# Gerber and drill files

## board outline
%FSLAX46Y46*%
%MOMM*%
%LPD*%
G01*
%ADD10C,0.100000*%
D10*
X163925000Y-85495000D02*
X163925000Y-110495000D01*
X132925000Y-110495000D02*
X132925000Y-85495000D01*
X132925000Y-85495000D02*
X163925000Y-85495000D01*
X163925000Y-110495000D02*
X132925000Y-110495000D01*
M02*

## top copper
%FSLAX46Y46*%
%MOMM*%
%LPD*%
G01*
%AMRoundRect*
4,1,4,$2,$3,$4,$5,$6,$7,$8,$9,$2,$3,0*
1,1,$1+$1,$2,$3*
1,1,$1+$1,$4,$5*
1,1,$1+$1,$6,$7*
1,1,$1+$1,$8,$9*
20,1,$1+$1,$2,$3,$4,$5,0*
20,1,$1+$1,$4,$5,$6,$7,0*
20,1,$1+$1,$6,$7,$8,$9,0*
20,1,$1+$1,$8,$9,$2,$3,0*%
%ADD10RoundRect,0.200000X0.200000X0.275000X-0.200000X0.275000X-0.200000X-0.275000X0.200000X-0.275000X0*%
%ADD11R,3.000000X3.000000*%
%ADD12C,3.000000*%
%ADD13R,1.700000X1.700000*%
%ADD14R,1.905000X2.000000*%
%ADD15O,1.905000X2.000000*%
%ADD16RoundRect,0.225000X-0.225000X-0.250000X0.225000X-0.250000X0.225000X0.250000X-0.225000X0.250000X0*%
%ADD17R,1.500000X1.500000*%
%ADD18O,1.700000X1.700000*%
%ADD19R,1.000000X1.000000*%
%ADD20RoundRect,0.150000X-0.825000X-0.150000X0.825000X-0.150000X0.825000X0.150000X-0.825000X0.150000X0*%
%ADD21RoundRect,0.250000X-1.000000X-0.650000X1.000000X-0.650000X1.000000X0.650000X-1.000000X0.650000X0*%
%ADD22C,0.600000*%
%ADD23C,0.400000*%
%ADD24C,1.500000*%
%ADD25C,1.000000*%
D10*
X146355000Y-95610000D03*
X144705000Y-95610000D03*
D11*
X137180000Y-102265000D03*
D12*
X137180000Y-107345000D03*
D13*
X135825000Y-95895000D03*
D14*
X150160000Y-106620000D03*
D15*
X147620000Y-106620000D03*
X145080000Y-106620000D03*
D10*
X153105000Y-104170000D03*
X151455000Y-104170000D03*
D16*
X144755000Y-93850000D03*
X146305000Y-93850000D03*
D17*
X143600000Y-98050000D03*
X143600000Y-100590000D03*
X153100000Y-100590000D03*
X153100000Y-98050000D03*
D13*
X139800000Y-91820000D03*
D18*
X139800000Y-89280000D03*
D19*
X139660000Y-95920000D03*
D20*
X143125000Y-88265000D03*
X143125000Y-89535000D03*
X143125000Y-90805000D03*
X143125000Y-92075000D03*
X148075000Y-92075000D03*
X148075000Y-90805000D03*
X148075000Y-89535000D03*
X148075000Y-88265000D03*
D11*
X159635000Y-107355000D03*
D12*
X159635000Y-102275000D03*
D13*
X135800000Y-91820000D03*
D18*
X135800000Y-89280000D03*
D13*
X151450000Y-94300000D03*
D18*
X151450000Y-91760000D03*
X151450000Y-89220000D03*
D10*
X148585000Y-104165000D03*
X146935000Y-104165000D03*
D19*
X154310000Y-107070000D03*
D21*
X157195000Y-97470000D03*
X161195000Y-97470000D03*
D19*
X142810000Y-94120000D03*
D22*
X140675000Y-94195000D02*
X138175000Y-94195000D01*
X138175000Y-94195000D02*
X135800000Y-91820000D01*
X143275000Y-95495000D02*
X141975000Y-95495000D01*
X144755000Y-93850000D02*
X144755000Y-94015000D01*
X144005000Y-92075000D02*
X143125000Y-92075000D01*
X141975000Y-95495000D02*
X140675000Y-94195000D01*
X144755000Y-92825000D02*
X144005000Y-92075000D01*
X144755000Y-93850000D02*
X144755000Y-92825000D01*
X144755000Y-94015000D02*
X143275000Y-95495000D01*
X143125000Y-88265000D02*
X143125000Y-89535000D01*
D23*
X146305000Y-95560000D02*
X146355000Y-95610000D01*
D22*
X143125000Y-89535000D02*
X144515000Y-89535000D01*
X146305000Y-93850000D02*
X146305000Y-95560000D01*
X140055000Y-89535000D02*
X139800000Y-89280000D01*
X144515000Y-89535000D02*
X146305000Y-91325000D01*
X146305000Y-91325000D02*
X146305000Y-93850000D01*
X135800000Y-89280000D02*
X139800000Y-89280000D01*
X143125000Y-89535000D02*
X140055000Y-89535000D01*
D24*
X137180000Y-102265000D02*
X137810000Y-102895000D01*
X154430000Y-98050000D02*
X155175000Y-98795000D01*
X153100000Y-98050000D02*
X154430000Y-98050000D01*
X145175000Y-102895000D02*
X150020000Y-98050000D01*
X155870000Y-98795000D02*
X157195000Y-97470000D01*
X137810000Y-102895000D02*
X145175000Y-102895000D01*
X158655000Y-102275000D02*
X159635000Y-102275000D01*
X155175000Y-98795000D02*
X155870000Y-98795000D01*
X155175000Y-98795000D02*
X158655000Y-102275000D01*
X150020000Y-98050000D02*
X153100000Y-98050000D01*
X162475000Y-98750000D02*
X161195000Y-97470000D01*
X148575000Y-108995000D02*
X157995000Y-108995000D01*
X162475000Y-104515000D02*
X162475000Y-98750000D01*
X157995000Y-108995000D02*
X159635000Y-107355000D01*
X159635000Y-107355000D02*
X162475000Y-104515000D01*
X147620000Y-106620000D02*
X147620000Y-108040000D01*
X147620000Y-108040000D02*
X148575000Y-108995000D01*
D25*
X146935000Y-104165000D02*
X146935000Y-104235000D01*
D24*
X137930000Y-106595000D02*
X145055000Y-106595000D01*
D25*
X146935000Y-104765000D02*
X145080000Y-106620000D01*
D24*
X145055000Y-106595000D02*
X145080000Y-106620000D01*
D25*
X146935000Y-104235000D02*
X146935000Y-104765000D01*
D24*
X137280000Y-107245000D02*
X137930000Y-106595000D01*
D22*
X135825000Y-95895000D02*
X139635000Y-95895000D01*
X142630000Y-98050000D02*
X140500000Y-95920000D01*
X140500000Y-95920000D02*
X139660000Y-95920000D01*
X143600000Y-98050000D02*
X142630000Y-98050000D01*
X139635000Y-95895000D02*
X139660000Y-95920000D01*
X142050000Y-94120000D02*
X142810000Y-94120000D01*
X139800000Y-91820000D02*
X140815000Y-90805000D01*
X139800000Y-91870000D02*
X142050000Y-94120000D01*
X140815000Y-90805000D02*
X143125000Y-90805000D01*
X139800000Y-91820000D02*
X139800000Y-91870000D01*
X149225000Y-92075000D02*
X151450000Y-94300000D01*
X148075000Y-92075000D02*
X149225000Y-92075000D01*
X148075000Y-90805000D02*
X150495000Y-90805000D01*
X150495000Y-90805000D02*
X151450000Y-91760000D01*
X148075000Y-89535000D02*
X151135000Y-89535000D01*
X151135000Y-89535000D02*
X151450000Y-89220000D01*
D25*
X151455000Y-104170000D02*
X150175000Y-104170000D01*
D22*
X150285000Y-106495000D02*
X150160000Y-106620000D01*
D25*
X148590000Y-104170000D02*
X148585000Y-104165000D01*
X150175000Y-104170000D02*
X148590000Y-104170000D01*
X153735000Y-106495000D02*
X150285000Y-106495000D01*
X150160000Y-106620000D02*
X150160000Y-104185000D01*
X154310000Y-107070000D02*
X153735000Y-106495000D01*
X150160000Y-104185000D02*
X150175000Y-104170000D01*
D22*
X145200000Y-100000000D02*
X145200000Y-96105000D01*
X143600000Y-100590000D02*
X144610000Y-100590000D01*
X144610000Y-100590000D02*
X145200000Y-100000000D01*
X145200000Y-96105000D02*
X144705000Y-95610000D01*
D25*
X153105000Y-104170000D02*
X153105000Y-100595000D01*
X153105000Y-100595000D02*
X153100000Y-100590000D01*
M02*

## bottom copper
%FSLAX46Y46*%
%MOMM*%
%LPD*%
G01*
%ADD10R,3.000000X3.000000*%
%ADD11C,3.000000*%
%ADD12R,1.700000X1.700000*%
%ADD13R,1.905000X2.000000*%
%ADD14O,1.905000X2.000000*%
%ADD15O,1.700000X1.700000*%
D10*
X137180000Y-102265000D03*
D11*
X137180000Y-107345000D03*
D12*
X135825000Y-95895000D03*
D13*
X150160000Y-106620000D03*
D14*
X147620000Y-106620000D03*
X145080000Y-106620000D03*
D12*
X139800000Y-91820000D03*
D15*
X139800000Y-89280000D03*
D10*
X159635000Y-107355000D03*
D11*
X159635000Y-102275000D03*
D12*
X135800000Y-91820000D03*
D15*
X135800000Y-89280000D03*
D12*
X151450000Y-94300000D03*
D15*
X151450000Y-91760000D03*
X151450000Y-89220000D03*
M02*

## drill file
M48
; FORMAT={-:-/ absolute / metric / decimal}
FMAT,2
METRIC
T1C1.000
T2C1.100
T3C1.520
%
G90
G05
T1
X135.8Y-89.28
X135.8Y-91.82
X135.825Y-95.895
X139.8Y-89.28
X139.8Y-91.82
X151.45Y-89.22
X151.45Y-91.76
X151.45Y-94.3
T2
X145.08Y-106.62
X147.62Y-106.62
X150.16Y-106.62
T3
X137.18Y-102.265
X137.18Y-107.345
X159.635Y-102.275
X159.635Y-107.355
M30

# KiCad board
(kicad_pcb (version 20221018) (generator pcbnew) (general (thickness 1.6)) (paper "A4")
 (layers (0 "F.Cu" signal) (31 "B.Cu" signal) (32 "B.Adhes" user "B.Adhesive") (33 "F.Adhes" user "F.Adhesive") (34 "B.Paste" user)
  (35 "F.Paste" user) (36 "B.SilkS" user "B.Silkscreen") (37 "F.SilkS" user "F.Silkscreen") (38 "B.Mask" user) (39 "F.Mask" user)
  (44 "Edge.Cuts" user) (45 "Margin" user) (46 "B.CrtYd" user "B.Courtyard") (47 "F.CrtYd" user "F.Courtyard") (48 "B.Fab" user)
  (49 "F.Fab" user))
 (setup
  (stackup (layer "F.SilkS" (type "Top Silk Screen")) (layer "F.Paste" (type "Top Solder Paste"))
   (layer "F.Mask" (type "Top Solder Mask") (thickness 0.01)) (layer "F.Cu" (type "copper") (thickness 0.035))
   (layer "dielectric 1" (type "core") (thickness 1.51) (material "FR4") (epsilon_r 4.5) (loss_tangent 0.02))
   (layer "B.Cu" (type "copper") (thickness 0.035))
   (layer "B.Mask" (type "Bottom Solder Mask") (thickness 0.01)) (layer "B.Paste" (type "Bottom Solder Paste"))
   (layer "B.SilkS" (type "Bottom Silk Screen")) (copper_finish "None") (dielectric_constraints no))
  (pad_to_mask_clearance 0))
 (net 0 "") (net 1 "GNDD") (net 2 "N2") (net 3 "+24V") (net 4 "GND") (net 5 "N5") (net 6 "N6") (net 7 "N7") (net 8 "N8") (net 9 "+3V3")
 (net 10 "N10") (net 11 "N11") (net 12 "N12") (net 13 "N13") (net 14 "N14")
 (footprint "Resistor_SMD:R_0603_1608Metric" (layer "F.Cu") (at 145.53 95.61 180)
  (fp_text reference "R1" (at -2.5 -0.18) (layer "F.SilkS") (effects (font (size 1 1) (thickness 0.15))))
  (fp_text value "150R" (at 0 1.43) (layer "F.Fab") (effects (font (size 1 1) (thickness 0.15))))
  (pad "1" smd roundrect (at -0.825 0 180) (size 0.8 0.95) (layers "F.Cu" "F.Paste" "F.Mask") (roundrect_rratio 0.25) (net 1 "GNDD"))
  (pad "2" smd roundrect (at 0.825 0 180) (size 0.8 0.95) (layers "F.Cu" "F.Paste" "F.Mask") (roundrect_rratio 0.25) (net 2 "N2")))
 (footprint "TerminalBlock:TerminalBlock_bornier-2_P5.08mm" (layer "F.Cu") (at 137.18 102.265 -90)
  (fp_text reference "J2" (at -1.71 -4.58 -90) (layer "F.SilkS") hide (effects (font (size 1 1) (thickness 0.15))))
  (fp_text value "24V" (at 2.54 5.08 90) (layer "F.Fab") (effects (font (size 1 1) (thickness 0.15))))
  (pad "1" thru_hole rect (at 0 0 270) (size 3 3) (drill 1.52) (layers "*.Cu" "*.Mask") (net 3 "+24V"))
  (pad "2" thru_hole circle (at 5.08 0 270) (size 3 3) (drill 1.52) (layers "*.Cu" "*.Mask") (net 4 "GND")))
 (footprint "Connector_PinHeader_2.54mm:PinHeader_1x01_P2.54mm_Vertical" (layer "F.Cu") (at 135.825 95.895)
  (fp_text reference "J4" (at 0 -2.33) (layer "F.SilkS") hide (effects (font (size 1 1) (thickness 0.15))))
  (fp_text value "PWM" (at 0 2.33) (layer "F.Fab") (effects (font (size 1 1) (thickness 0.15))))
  (pad "1" thru_hole rect (at 0 0) (size 1.7 1.7) (drill 1) (layers "*.Cu" "*.Mask") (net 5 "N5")))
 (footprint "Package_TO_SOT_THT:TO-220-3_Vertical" (layer "F.Cu") (at 150.16 106.62 180)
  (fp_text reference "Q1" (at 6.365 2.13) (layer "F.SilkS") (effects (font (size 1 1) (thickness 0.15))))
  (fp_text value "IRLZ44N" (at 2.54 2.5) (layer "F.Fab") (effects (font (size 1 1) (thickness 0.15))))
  (pad "1" thru_hole rect (at 0 0 180) (size 1.905 2) (drill 1.1) (layers "*.Cu" "*.Mask") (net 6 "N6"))
  (pad "2" thru_hole oval (at 2.54 0 180) (size 1.905 2) (drill 1.1) (layers "*.Cu" "*.Mask") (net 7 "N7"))
  (pad "3" thru_hole oval (at 5.08 0 180) (size 1.905 2) (drill 1.1) (layers "*.Cu" "*.Mask") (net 4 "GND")))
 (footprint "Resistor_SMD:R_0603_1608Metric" (layer "F.Cu") (at 152.28 104.17 180)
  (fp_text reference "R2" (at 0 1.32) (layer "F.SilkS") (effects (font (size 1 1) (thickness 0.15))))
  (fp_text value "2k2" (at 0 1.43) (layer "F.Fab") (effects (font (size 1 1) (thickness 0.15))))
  (pad "1" smd roundrect (at -0.825 0 180) (size 0.8 0.95) (layers "F.Cu" "F.Paste" "F.Mask") (roundrect_rratio 0.25) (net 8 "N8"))
  (pad "2" smd roundrect (at 0.825 0 180) (size 0.8 0.95) (layers "F.Cu" "F.Paste" "F.Mask") (roundrect_rratio 0.25) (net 6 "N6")))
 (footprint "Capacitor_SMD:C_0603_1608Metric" (layer "F.Cu") (at 145.53 93.85)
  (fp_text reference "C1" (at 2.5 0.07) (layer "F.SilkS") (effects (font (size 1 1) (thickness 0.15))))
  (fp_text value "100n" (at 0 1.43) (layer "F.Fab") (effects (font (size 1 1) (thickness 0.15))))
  (pad "1" smd roundrect (at -0.775 0) (size 0.9 0.95) (layers "F.Cu" "F.Paste" "F.Mask") (roundrect_rratio 0.25) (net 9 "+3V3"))
  (pad "2" smd roundrect (at 0.775 0) (size 0.9 0.95) (layers "F.Cu" "F.Paste" "F.Mask") (roundrect_rratio 0.25) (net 1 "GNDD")))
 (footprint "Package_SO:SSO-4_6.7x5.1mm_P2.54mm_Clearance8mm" (layer "F.Cu") (at 148.35 99.32)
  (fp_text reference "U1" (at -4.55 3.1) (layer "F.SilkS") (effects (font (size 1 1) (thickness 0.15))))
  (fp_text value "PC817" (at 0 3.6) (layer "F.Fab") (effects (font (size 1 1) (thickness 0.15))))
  (pad "1" smd rect (at -4.75 -1.27) (size 1.5 1.5) (layers "F.Cu" "F.Paste" "F.Mask") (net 5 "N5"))
  (pad "2" smd rect (at -4.75 1.27) (size 1.5 1.5) (layers "F.Cu" "F.Paste" "F.Mask") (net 2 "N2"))
  (pad "3" smd rect (at 4.75 1.27) (size 1.5 1.5) (layers "F.Cu" "F.Paste" "F.Mask") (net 8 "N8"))
  (pad "4" smd rect (at 4.75 -1.27) (size 1.5 1.5) (layers "F.Cu" "F.Paste" "F.Mask") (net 3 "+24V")))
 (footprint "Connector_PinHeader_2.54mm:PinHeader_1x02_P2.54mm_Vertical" (layer "F.Cu") (at 139.8 91.82 180)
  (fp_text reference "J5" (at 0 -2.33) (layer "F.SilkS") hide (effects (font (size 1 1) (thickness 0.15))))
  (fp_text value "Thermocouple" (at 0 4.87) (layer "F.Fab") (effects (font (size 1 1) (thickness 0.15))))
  (pad "1" thru_hole rect (at 0 0 180) (size 1.7 1.7) (drill 1) (layers "*.Cu" "*.Mask") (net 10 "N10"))
  (pad "2" thru_hole oval (at 0 2.54 180) (size 1.7 1.7) (drill 1) (layers "*.Cu" "*.Mask") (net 1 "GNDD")))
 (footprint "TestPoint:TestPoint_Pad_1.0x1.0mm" (layer "F.Cu") (at 139.66 95.92)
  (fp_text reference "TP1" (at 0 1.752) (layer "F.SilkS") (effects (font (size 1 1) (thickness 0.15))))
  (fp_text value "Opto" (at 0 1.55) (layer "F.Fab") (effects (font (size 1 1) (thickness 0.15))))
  (pad "1" smd rect (at 0 0) (size 1 1) (layers "F.Cu" "F.Mask") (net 5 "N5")))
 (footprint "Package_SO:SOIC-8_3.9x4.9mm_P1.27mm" (layer "F.Cu") (at 145.6 90.17)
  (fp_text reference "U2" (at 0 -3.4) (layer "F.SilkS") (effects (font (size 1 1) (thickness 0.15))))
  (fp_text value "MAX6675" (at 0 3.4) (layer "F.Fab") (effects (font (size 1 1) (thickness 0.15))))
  (pad "1" smd roundrect (at -2.475 -1.905) (size 1.95 0.6) (layers "F.Cu" "F.Paste" "F.Mask") (roundrect_rratio 0.25) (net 1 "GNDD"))
  (pad "2" smd roundrect (at -2.475 -0.635) (size 1.95 0.6) (layers "F.Cu" "F.Paste" "F.Mask") (roundrect_rratio 0.25) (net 1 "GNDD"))
  (pad "3" smd roundrect (at -2.475 0.635) (size 1.95 0.6) (layers "F.Cu" "F.Paste" "F.Mask") (roundrect_rratio 0.25) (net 10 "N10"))
  (pad "4" smd roundrect (at -2.475 1.905) (size 1.95 0.6) (layers "F.Cu" "F.Paste" "F.Mask") (roundrect_rratio 0.25) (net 9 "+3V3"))
  (pad "5" smd roundrect (at 2.475 1.905) (size 1.95 0.6) (layers "F.Cu" "F.Paste" "F.Mask") (roundrect_rratio 0.25) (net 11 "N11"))
  (pad "6" smd roundrect (at 2.475 0.635) (size 1.95 0.6) (layers "F.Cu" "F.Paste" "F.Mask") (roundrect_rratio 0.25) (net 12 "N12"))
  (pad "7" smd roundrect (at 2.475 -0.635) (size 1.95 0.6) (layers "F.Cu" "F.Paste" "F.Mask") (roundrect_rratio 0.25) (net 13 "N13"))
  (pad "8" smd roundrect (at 2.475 -1.905) (size 1.95 0.6) (layers "F.Cu" "F.Paste" "F.Mask") (roundrect_rratio 0.25) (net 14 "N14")))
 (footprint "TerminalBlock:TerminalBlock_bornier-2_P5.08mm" (layer "F.Cu") (at 159.635 107.355 90)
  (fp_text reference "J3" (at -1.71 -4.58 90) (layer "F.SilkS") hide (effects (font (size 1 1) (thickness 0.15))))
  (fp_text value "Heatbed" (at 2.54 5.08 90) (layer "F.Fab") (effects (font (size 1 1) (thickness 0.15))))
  (pad "1" thru_hole rect (at 0 0 90) (size 3 3) (drill 1.52) (layers "*.Cu" "*.Mask") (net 7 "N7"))
  (pad "2" thru_hole circle (at 5.08 0 90) (size 3 3) (drill 1.52) (layers "*.Cu" "*.Mask") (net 3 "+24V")))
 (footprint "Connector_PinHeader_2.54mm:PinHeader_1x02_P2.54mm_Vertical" (layer "F.Cu") (at 135.8 91.82 180)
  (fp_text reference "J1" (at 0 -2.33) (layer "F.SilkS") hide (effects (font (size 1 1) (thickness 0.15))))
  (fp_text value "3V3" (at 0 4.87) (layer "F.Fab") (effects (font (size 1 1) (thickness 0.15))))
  (pad "1" thru_hole rect (at 0 0 180) (size 1.7 1.7) (drill 1) (layers "*.Cu" "*.Mask") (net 9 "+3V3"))
  (pad "2" thru_hole oval (at 0 2.54 180) (size 1.7 1.7) (drill 1) (layers "*.Cu" "*.Mask") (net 1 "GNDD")))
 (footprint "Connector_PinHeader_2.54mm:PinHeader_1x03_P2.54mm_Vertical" (layer "F.Cu") (at 151.45 94.3 180)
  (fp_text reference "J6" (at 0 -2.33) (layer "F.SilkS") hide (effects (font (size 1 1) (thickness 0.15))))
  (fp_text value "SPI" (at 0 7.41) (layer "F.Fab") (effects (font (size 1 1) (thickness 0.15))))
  (pad "1" thru_hole rect (at 0 0 180) (size 1.7 1.7) (drill 1) (layers "*.Cu" "*.Mask") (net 11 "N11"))
  (pad "2" thru_hole oval (at 0 2.54 180) (size 1.7 1.7) (drill 1) (layers "*.Cu" "*.Mask") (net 12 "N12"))
  (pad "3" thru_hole oval (at 0 5.08 180) (size 1.7 1.7) (drill 1) (layers "*.Cu" "*.Mask") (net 13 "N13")))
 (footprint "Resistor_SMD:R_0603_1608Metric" (layer "F.Cu") (at 147.76 104.165 180)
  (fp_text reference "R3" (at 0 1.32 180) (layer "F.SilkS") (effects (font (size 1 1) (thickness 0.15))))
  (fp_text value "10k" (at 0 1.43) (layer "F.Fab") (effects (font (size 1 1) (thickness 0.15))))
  (pad "1" smd roundrect (at -0.825 0 180) (size 0.8 0.95) (layers "F.Cu" "F.Paste" "F.Mask") (roundrect_rratio 0.25) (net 6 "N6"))
  (pad "2" smd roundrect (at 0.825 0 180) (size 0.8 0.95) (layers "F.Cu" "F.Paste" "F.Mask") (roundrect_rratio 0.25) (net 4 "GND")))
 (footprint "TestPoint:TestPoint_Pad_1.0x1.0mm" (layer "F.Cu") (at 154.31 107.07)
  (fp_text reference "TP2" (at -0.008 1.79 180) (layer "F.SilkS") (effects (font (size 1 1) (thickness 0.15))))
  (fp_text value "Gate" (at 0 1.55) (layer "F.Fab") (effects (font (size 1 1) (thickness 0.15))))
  (pad "1" smd rect (at 0 0) (size 1 1) (layers "F.Cu" "F.Mask") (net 6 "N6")))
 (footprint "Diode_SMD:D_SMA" (layer "F.Cu") (at 159.195 97.47)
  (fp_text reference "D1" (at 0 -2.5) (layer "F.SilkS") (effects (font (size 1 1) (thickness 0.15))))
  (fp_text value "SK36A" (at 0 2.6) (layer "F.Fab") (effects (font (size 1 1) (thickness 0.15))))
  (pad "1" smd roundrect (at -2 0) (size 2.5 1.8) (layers "F.Cu" "F.Paste" "F.Mask") (roundrect_rratio 0.1388888889) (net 3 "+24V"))
  (pad "2" smd roundrect (at 2 0) (size 2.5 1.8) (layers "F.Cu" "F.Paste" "F.Mask") (roundrect_rratio 0.1388888889) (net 7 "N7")))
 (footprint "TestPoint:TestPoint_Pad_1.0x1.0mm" (layer "F.Cu") (at 142.81 94.12 180)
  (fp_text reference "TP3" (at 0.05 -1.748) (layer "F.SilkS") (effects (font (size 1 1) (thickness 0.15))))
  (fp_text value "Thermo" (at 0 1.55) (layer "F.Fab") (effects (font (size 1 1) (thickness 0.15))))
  (pad "1" smd rect (at 0 0 180) (size 1 1) (layers "F.Cu" "F.Mask") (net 10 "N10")))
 (gr_line (start 163.925 85.495) (end 163.925 110.495) (stroke (width 0.1) (type default)) (layer "Edge.Cuts"))
 (gr_line (start 132.925 110.495) (end 132.925 85.495) (stroke (width 0.1) (type default)) (layer "Edge.Cuts"))
 (gr_line (start 132.925 85.495) (end 163.925 85.495) (stroke (width 0.1) (type default)) (layer "Edge.Cuts"))
 (gr_line (start 163.925 110.495) (end 132.925 110.495) (stroke (width 0.1) (type default)) (layer "Edge.Cuts"))
 (segment (start 140.675 94.195) (end 138.175 94.195) (width 0.6) (layer "F.Cu") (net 9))
 (segment (start 138.175 94.195) (end 135.8 91.82) (width 0.6) (layer "F.Cu") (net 9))
 (segment (start 143.275 95.495) (end 141.975 95.495) (width 0.6) (layer "F.Cu") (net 9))
 (segment (start 144.755 93.85) (end 144.755 94.015) (width 0.6) (layer "F.Cu") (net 9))
 (segment (start 144.005 92.075) (end 143.125 92.075) (width 0.6) (layer "F.Cu") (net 9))
 (segment (start 141.975 95.495) (end 140.675 94.195) (width 0.6) (layer "F.Cu") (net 9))
 (segment (start 144.755 92.825) (end 144.005 92.075) (width 0.6) (layer "F.Cu") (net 9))
 (segment (start 144.755 93.85) (end 144.755 92.825) (width 0.6) (layer "F.Cu") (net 9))
 (segment (start 144.755 94.015) (end 143.275 95.495) (width 0.6) (layer "F.Cu") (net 9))
 (segment (start 143.125 88.265) (end 143.125 89.535) (width 0.6) (layer "F.Cu") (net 1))
 (segment (start 146.305 95.56) (end 146.355 95.61) (width 0.4) (layer "F.Cu") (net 1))
 (segment (start 143.125 89.535) (end 144.515 89.535) (width 0.6) (layer "F.Cu") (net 1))
 (segment (start 146.305 93.85) (end 146.305 95.56) (width 0.6) (layer "F.Cu") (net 1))
 (segment (start 140.055 89.535) (end 139.8 89.28) (width 0.6) (layer "F.Cu") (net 1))
 (segment (start 144.515 89.535) (end 146.305 91.325) (width 0.6) (layer "F.Cu") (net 1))
 (segment (start 146.305 91.325) (end 146.305 93.85) (width 0.6) (layer "F.Cu") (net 1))
 (segment (start 135.8 89.28) (end 139.8 89.28) (width 0.6) (layer "F.Cu") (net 1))
 (segment (start 143.125 89.535) (end 140.055 89.535) (width 0.6) (layer "F.Cu") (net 1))
 (segment (start 137.18 102.265) (end 137.81 102.895) (width 1.5) (layer "F.Cu") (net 3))
 (segment (start 154.43 98.05) (end 155.175 98.795) (width 1.5) (layer "F.Cu") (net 3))
 (segment (start 153.1 98.05) (end 154.43 98.05) (width 1.5) (layer "F.Cu") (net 3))
 (segment (start 145.175 102.895) (end 150.02 98.05) (width 1.5) (layer "F.Cu") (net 3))
 (segment (start 155.87 98.795) (end 157.195 97.47) (width 1.5) (layer "F.Cu") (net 3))
 (segment (start 137.81 102.895) (end 145.175 102.895) (width 1.5) (layer "F.Cu") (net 3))
 (segment (start 158.655 102.275) (end 159.635 102.275) (width 1.5) (layer "F.Cu") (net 3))
 (segment (start 155.175 98.795) (end 155.87 98.795) (width 1.5) (layer "F.Cu") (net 3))
 (segment (start 155.175 98.795) (end 158.655 102.275) (width 1.5) (layer "F.Cu") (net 3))
 (segment (start 150.02 98.05) (end 153.1 98.05) (width 1.5) (layer "F.Cu") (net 3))
 (segment (start 162.475 98.75) (end 161.195 97.47) (width 1.5) (layer "F.Cu") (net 7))
 (segment (start 148.575 108.995) (end 157.995 108.995) (width 1.5) (layer "F.Cu") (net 7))
 (segment (start 162.475 104.515) (end 162.475 98.75) (width 1.5) (layer "F.Cu") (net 7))
 (segment (start 157.995 108.995) (end 159.635 107.355) (width 1.5) (layer "F.Cu") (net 7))
 (segment (start 159.635 107.355) (end 162.475 104.515) (width 1.5) (layer "F.Cu") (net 7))
 (segment (start 147.62 106.62) (end 147.62 108.04) (width 1.5) (layer "F.Cu") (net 7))
 (segment (start 147.62 108.04) (end 148.575 108.995) (width 1.5) (layer "F.Cu") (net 7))
 (segment (start 146.935 104.165) (end 146.935 104.235) (width 1) (layer "F.Cu") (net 4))
 (segment (start 137.93 106.595) (end 145.055 106.595) (width 1.5) (layer "F.Cu") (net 4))
 (segment (start 146.935 104.765) (end 145.08 106.62) (width 1) (layer "F.Cu") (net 4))
 (segment (start 145.055 106.595) (end 145.08 106.62) (width 1.5) (layer "F.Cu") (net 4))
 (segment (start 146.935 104.235) (end 146.935 104.765) (width 1) (layer "F.Cu") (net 4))
 (segment (start 137.28 107.245) (end 137.93 106.595) (width 1.5) (layer "F.Cu") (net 4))
 (segment (start 135.825 95.895) (end 139.635 95.895) (width 0.6) (layer "F.Cu") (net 5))
 (segment (start 142.63 98.05) (end 140.5 95.92) (width 0.6) (layer "F.Cu") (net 5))
 (segment (start 140.5 95.92) (end 139.66 95.92) (width 0.6) (layer "F.Cu") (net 5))
 (segment (start 143.6 98.05) (end 142.63 98.05) (width 0.6) (layer "F.Cu") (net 5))
 (segment (start 139.635 95.895) (end 139.66 95.92) (width 0.6) (layer "F.Cu") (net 5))
 (segment (start 142.05 94.12) (end 142.81 94.12) (width 0.6) (layer "F.Cu") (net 10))
 (segment (start 139.8 91.82) (end 140.815 90.805) (width 0.6) (layer "F.Cu") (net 10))
 (segment (start 139.8 91.87) (end 142.05 94.12) (width 0.6) (layer "F.Cu") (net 10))
 (segment (start 140.815 90.805) (end 143.125 90.805) (width 0.6) (layer "F.Cu") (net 10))
 (segment (start 139.8 91.82) (end 139.8 91.87) (width 0.6) (layer "F.Cu") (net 10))
 (segment (start 149.225 92.075) (end 151.45 94.3) (width 0.6) (layer "F.Cu") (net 11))
 (segment (start 148.075 92.075) (end 149.225 92.075) (width 0.6) (layer "F.Cu") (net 11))
 (segment (start 148.075 90.805) (end 150.495 90.805) (width 0.6) (layer "F.Cu") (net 12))
 (segment (start 150.495 90.805) (end 151.45 91.76) (width 0.6) (layer "F.Cu") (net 12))
 (segment (start 148.075 89.535) (end 151.135 89.535) (width 0.6) (layer "F.Cu") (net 13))
 (segment (start 151.135 89.535) (end 151.45 89.22) (width 0.6) (layer "F.Cu") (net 13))
 (segment (start 151.455 104.17) (end 150.175 104.17) (width 1) (layer "F.Cu") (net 6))
 (segment (start 150.285 106.495) (end 150.16 106.62) (width 0.6) (layer "F.Cu") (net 6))
 (segment (start 148.59 104.17) (end 148.585 104.165) (width 1) (layer "F.Cu") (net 6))
 (segment (start 150.175 104.17) (end 148.59 104.17) (width 1) (layer "F.Cu") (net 6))
 (segment (start 153.735 106.495) (end 150.285 106.495) (width 1) (layer "F.Cu") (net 6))
 (segment (start 150.16 106.62) (end 150.16 104.185) (width 1) (layer "F.Cu") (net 6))
 (segment (start 154.31 107.07) (end 153.735 106.495) (width 1) (layer "F.Cu") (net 6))
 (segment (start 150.16 104.185) (end 150.175 104.17) (width 1) (layer "F.Cu") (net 6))
 (segment (start 145.2 100) (end 145.2 96.105) (width 0.6) (layer "F.Cu") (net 2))
 (segment (start 143.6 100.59) (end 144.61 100.59) (width 0.6) (layer "F.Cu") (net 2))
 (segment (start 144.61 100.59) (end 145.2 100) (width 0.6) (layer "F.Cu") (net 2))
 (segment (start 145.2 96.105) (end 144.705 95.61) (width 0.6) (layer "F.Cu") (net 2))
 (segment (start 153.105 104.17) (end 153.105 100.595) (width 1) (layer "F.Cu") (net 8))
 (segment (start 153.105 100.595) (end 153.1 100.59) (width 1) (layer "F.Cu") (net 8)))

